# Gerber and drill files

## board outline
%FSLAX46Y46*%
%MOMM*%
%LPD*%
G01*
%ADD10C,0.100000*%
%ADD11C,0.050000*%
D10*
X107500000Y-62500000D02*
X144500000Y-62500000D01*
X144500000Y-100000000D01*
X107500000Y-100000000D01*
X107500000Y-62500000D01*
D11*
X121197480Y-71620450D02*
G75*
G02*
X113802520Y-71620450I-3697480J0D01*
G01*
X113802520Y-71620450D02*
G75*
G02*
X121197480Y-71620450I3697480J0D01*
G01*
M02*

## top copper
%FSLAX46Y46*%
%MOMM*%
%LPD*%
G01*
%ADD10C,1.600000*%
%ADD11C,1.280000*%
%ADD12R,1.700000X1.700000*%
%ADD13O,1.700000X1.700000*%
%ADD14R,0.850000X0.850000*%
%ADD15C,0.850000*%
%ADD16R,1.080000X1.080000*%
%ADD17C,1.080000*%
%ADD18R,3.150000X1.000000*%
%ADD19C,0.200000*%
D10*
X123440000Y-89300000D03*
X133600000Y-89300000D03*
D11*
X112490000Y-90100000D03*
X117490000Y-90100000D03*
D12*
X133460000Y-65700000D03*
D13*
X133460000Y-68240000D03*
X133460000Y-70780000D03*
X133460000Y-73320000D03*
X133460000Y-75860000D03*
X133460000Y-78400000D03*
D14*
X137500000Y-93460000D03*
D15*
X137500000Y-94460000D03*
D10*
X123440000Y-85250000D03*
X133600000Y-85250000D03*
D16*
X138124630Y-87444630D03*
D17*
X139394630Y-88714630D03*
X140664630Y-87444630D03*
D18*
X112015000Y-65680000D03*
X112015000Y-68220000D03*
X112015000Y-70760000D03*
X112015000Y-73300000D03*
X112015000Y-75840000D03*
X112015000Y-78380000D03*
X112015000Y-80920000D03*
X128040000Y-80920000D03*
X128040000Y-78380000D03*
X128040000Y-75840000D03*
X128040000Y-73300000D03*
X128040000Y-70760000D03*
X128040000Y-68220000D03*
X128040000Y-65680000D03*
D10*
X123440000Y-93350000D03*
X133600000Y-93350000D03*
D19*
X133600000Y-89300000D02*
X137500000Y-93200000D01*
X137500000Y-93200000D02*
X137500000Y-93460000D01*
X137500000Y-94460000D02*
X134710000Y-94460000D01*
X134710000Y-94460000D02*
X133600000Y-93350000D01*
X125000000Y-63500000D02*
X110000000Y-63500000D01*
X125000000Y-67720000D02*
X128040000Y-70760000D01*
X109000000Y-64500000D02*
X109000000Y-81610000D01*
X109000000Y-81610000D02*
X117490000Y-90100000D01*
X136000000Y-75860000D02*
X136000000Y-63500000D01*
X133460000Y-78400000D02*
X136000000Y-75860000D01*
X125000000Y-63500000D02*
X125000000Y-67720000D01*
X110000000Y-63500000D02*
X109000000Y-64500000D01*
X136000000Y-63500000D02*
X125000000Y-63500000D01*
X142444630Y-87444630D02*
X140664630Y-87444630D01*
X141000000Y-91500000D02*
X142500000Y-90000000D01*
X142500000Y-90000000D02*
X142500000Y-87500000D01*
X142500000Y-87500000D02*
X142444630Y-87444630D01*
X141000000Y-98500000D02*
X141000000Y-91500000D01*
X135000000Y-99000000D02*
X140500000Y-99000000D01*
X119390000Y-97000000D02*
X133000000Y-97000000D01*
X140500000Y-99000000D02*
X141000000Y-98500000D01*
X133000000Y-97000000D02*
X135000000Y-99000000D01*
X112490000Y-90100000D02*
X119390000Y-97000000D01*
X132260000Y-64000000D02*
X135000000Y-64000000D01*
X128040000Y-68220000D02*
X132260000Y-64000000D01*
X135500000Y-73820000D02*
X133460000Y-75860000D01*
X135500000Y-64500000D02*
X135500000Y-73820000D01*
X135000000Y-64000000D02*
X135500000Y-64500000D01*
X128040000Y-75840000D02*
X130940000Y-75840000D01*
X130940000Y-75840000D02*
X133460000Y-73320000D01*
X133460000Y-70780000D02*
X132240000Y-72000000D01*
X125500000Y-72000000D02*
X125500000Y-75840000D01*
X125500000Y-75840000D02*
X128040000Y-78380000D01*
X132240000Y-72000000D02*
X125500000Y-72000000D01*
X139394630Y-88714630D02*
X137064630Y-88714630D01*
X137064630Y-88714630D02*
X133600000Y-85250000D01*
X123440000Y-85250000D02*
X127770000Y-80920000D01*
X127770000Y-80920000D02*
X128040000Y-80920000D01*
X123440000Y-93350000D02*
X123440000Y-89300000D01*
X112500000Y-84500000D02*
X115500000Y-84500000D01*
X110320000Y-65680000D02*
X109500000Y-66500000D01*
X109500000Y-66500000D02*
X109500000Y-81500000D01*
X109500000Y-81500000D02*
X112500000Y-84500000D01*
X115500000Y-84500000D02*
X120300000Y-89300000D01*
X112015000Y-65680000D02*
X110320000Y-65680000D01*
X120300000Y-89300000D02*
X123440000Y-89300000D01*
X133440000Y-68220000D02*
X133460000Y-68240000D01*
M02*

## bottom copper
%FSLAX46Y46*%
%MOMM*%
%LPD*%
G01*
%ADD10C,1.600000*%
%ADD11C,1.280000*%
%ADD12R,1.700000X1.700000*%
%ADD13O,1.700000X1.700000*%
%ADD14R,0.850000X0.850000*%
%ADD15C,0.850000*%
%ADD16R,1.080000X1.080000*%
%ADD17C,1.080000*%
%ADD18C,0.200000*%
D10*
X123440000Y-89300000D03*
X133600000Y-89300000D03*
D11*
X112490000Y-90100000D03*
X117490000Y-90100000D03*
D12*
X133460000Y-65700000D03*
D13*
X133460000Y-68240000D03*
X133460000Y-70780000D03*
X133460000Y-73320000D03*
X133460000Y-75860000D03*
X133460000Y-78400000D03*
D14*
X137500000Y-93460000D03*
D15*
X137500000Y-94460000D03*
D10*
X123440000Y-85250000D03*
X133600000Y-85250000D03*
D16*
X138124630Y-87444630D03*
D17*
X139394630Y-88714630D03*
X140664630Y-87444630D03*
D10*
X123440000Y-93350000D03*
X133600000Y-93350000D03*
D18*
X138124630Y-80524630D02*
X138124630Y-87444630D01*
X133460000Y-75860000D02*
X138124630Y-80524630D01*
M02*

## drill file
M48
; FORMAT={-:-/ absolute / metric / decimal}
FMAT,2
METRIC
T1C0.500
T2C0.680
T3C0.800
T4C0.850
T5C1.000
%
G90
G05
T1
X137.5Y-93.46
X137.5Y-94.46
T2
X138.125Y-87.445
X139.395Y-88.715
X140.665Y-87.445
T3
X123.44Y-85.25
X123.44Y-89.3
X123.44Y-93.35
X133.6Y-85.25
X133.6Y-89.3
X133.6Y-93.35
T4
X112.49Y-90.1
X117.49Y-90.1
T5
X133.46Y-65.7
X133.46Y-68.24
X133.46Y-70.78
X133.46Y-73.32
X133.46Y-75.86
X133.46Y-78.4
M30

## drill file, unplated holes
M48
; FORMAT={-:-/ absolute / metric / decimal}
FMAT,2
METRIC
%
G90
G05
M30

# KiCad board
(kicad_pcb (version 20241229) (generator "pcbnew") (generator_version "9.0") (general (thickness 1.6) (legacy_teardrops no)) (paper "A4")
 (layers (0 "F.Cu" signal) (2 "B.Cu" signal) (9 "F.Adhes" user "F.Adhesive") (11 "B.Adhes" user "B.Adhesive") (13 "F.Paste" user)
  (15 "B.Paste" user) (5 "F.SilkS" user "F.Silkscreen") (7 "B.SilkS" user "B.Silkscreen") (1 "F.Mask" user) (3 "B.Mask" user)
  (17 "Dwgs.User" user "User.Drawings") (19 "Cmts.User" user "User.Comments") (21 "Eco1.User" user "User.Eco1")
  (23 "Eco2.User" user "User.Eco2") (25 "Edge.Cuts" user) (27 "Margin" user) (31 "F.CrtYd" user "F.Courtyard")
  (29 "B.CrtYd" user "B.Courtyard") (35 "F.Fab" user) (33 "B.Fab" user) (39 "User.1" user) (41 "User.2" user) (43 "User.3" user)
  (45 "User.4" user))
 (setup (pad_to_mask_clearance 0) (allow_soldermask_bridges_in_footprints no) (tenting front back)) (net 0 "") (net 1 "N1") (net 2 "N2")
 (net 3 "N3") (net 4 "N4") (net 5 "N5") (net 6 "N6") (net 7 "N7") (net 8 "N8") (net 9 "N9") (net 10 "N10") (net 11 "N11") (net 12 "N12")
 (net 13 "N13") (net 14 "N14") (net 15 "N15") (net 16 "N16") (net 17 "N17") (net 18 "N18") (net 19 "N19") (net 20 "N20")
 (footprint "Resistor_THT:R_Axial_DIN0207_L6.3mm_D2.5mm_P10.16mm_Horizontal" (layer "F.Cu") (at 123.44 89.3)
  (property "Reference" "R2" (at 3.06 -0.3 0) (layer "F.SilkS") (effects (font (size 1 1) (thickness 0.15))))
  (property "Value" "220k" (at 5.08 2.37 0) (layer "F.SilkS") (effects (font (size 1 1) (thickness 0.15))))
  (pad "1" thru_hole circle (at 0 0) (size 1.6 1.6) (drill 0.8) (layers "*.Cu" "*.Mask") (remove_unused_layers no) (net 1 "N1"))
  (pad "2" thru_hole circle (at 10.16 0) (size 1.6 1.6) (drill 0.8) (layers "*.Cu" "*.Mask") (remove_unused_layers no) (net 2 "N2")))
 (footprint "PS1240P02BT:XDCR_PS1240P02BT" (layer "F.Cu") (at 114.99 90.1)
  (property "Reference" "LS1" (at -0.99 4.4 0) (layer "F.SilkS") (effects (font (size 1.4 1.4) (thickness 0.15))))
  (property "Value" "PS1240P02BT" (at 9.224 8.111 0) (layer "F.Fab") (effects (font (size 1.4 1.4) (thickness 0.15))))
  (pad "1" thru_hole circle (at -2.5 0) (size 1.28 1.28) (drill 0.85) (layers "*.Cu" "*.Mask") (remove_unused_layers no) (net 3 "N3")
   (solder_mask_margin 0.102))
  (pad "2" thru_hole circle (at 2.5 0) (size 1.28 1.28) (drill 0.85) (layers "*.Cu" "*.Mask") (remove_unused_layers no) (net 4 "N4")
   (solder_mask_margin 0.102)))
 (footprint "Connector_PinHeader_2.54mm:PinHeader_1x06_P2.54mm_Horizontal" (layer "F.Cu") (at 133.46 65.7)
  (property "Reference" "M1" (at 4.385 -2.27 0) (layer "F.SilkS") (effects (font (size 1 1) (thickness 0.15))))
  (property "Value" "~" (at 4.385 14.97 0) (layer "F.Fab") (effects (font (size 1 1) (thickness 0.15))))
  (pad "1" thru_hole rect (at 0 0) (size 1.7 1.7) (drill 1) (layers "*.Cu" "*.Mask") (remove_unused_layers no) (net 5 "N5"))
  (pad "2" thru_hole oval (at 0 2.54) (size 1.7 1.7) (drill 1) (layers "*.Cu" "*.Mask") (remove_unused_layers no) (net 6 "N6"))
  (pad "3" thru_hole oval (at 0 5.08) (size 1.7 1.7) (drill 1) (layers "*.Cu" "*.Mask") (remove_unused_layers no) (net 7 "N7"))
  (pad "4" thru_hole oval (at 0 7.62) (size 1.7 1.7) (drill 1) (layers "*.Cu" "*.Mask") (remove_unused_layers no) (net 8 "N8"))
  (pad "5" thru_hole oval (at 0 10.16) (size 1.7 1.7) (drill 1) (layers "*.Cu" "*.Mask") (remove_unused_layers no) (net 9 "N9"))
  (pad "6" thru_hole oval (at 0 12.7) (size 1.7 1.7) (drill 1) (layers "*.Cu" "*.Mask") (remove_unused_layers no) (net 4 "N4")))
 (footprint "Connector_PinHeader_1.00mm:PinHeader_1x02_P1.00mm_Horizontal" (layer "F.Cu") (at 137.5 93.46)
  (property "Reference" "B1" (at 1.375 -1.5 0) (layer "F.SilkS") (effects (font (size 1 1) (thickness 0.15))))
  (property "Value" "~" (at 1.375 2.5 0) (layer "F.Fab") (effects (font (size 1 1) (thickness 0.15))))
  (pad "1" thru_hole rect (at 0 0) (size 0.85 0.85) (drill 0.5) (layers "*.Cu" "*.Mask") (remove_unused_layers no) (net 2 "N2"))
  (pad "2" thru_hole circle (at 0 1) (size 0.85 0.85) (drill 0.5) (layers "*.Cu" "*.Mask") (remove_unused_layers no) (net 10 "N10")))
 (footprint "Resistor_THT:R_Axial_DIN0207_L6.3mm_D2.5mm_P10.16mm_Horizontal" (layer "F.Cu") (at 123.44 85.25)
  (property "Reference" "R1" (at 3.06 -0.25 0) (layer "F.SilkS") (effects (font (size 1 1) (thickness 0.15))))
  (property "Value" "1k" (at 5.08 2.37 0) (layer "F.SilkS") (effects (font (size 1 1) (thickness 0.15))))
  (pad "1" thru_hole circle (at 0 0) (size 1.6 1.6) (drill 0.8) (layers "*.Cu" "*.Mask") (remove_unused_layers no) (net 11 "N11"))
  (pad "2" thru_hole circle (at 10.16 0) (size 1.6 1.6) (drill 0.8) (layers "*.Cu" "*.Mask") (remove_unused_layers no) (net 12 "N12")))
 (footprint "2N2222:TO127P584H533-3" (layer "F.Cu") (at 139.39463 87.44463)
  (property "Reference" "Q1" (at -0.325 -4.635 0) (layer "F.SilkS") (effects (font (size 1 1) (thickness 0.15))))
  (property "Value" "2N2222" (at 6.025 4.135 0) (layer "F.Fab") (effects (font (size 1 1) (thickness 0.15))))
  (pad "1" thru_hole rect (at -1.27 0) (size 1.08 1.08) (drill 0.68) (layers "*.Cu" "*.Mask") (remove_unused_layers no) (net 9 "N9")
   (solder_mask_margin 0.102))
  (pad "2" thru_hole circle (at 0 1.27) (size 1.08 1.08) (drill 0.68) (layers "*.Cu" "*.Mask") (remove_unused_layers no) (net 12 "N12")
   (solder_mask_margin 0.102))
  (pad "3" thru_hole circle (at 1.27 0 3) (size 1.08 1.08) (drill 0.68) (layers "*.Cu" "*.Mask") (remove_unused_layers no) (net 3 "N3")
   (solder_mask_margin 0.102)))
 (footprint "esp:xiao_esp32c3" (layer "F.Cu") (at 120.615 75.1)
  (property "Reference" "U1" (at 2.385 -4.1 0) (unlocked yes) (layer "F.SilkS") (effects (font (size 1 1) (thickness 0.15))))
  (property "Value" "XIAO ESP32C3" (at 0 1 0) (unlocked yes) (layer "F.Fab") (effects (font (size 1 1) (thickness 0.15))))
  (pad "1" smd rect (at -8.6 -9.42) (size 3.15 1) (layers "F.Cu" "F.Mask" "F.Paste") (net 1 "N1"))
  (pad "2" smd rect (at -8.6 -6.88) (size 3.15 1) (layers "F.Cu" "F.Mask" "F.Paste") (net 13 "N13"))
  (pad "3" smd rect (at -8.6 -4.34) (size 3.15 1) (layers "F.Cu" "F.Mask" "F.Paste") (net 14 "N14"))
  (pad "4" smd rect (at -8.6 -1.8) (size 3.15 1) (layers "F.Cu" "F.Mask" "F.Paste") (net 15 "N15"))
  (pad "5" smd rect (at -8.6 0.74) (size 3.15 1) (layers "F.Cu" "F.Mask" "F.Paste") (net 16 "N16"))
  (pad "6" smd rect (at -8.6 3.28) (size 3.15 1) (layers "F.Cu" "F.Mask" "F.Paste") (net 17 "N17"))
  (pad "7" smd rect (at -8.6 5.82) (size 3.15 1) (layers "F.Cu" "F.Mask" "F.Paste") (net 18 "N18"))
  (pad "8" smd rect (at 7.425 5.82) (size 3.15 1) (layers "F.Cu" "F.Mask" "F.Paste") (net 11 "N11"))
  (pad "9" smd rect (at 7.425 3.28) (size 3.15 1) (layers "F.Cu" "F.Mask" "F.Paste") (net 7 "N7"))
  (pad "10" smd rect (at 7.425 0.74) (size 3.15 1) (layers "F.Cu" "F.Mask" "F.Paste") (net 8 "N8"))
  (pad "11" smd rect (at 7.425 -1.8) (size 3.15 1) (layers "F.Cu" "F.Mask" "F.Paste") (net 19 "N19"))
  (pad "12" smd rect (at 7.425 -4.34) (size 3.15 1) (layers "F.Cu" "F.Mask" "F.Paste") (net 4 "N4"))
  (pad "13" smd rect (at 7.425 -6.88) (size 3.15 1) (layers "F.Cu" "F.Mask" "F.Paste") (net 9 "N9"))
  (pad "14" smd rect (at 7.425 -9.42) (size 3.15 1) (layers "F.Cu" "F.Mask" "F.Paste") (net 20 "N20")))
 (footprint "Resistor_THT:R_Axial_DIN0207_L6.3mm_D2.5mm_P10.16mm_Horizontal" (layer "F.Cu") (at 123.44 93.35)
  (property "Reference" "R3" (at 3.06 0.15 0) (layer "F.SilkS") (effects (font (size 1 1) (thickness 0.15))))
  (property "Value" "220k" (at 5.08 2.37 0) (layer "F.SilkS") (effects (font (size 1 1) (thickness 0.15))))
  (pad "1" thru_hole circle (at 0 0) (size 1.6 1.6) (drill 0.8) (layers "*.Cu" "*.Mask") (remove_unused_layers no) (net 1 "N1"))
  (pad "2" thru_hole circle (at 10.16 0) (size 1.6 1.6) (drill 0.8) (layers "*.Cu" "*.Mask") (remove_unused_layers no) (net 10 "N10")))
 (gr_rect (start 107.5 62.5) (end 144.5 100) (stroke (width 0.1) (type solid)) (fill no) (layer "Edge.Cuts"))
 (gr_circle (center 117.5 71.62045) (end 119 75) (stroke (width 0.05) (type default)) (fill no) (layer "Edge.Cuts"))
 (segment (start 133.6 89.3) (end 137.5 93.2) (width 0.2) (layer "F.Cu") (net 2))
 (segment (start 137.5 93.2) (end 137.5 93.46) (width 0.2) (layer "F.Cu") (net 2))
 (segment (start 137.5 94.46) (end 134.71 94.46) (width 0.2) (layer "F.Cu") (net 10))
 (segment (start 134.71 94.46) (end 133.6 93.35) (width 0.2) (layer "F.Cu") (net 10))
 (segment (start 125 63.5) (end 110 63.5) (width 0.2) (layer "F.Cu") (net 4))
 (segment (start 125 67.72) (end 128.04 70.76) (width 0.2) (layer "F.Cu") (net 4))
 (segment (start 109 64.5) (end 109 81.61) (width 0.2) (layer "F.Cu") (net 4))
 (segment (start 109 81.61) (end 117.49 90.1) (width 0.2) (layer "F.Cu") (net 4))
 (segment (start 136 75.86) (end 136 63.5) (width 0.2) (layer "F.Cu") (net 4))
 (segment (start 133.46 78.4) (end 136 75.86) (width 0.2) (layer "F.Cu") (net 4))
 (segment (start 125 63.5) (end 125 67.72) (width 0.2) (layer "F.Cu") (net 4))
 (segment (start 110 63.5) (end 109 64.5) (width 0.2) (layer "F.Cu") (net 4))
 (segment (start 136 63.5) (end 125 63.5) (width 0.2) (layer "F.Cu") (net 4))
 (segment (start 142.44463 87.44463) (end 140.66463 87.44463) (width 0.2) (layer "F.Cu") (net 3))
 (segment (start 141 91.5) (end 142.5 90) (width 0.2) (layer "F.Cu") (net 3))
 (segment (start 142.5 90) (end 142.5 87.5) (width 0.2) (layer "F.Cu") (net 3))
 (segment (start 142.5 87.5) (end 142.44463 87.44463) (width 0.2) (layer "F.Cu") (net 3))
 (segment (start 141 98.5) (end 141 91.5) (width 0.2) (layer "F.Cu") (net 3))
 (segment (start 135 99) (end 140.5 99) (width 0.2) (layer "F.Cu") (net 3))
 (segment (start 119.39 97) (end 133 97) (width 0.2) (layer "F.Cu") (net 3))
 (segment (start 140.5 99) (end 141 98.5) (width 0.2) (layer "F.Cu") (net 3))
 (segment (start 133 97) (end 135 99) (width 0.2) (layer "F.Cu") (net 3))
 (segment (start 112.49 90.1) (end 119.39 97) (width 0.2) (layer "F.Cu") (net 3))
 (segment (start 132.26 64) (end 135 64) (width 0.2) (layer "F.Cu") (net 9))
 (segment (start 128.04 68.22) (end 132.26 64) (width 0.2) (layer "F.Cu") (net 9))
 (segment (start 135.5 73.82) (end 133.46 75.86) (width 0.2) (layer "F.Cu") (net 9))
 (segment (start 135.5 64.5) (end 135.5 73.82) (width 0.2) (layer "F.Cu") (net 9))
 (segment (start 135 64) (end 135.5 64.5) (width 0.2) (layer "F.Cu") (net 9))
 (segment (start 138.12463 80.52463) (end 138.12463 87.44463) (width 0.2) (layer "B.Cu") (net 9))
 (segment (start 133.46 75.86) (end 138.12463 80.52463) (width 0.2) (layer "B.Cu") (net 9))
 (segment (start 128.04 75.84) (end 130.94 75.84) (width 0.2) (layer "F.Cu") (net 8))
 (segment (start 130.94 75.84) (end 133.46 73.32) (width 0.2) (layer "F.Cu") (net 8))
 (segment (start 133.46 70.78) (end 132.24 72) (width 0.2) (layer "F.Cu") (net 7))
 (segment (start 125.5 72) (end 125.5 75.84) (width 0.2) (layer "F.Cu") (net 7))
 (segment (start 125.5 75.84) (end 128.04 78.38) (width 0.2) (layer "F.Cu") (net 7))
 (segment (start 132.24 72) (end 125.5 72) (width 0.2) (layer "F.Cu") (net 7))
 (segment (start 139.39463 88.71463) (end 137.06463 88.71463) (width 0.2) (layer "F.Cu") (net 12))
 (segment (start 137.06463 88.71463) (end 133.6 85.25) (width 0.2) (layer "F.Cu") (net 12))
 (segment (start 123.44 85.25) (end 127.77 80.92) (width 0.2) (layer "F.Cu") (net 11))
 (segment (start 127.77 80.92) (end 128.04 80.92) (width 0.2) (layer "F.Cu") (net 11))
 (segment (start 123.44 93.35) (end 123.44 89.3) (width 0.2) (layer "F.Cu") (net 1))
 (segment (start 112.5 84.5) (end 115.5 84.5) (width 0.2) (layer "F.Cu") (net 1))
 (segment (start 110.32 65.68) (end 109.5 66.5) (width 0.2) (layer "F.Cu") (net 1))
 (segment (start 109.5 66.5) (end 109.5 81.5) (width 0.2) (layer "F.Cu") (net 1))
 (segment (start 109.5 81.5) (end 112.5 84.5) (width 0.2) (layer "F.Cu") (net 1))
 (segment (start 115.5 84.5) (end 120.3 89.3) (width 0.2) (layer "F.Cu") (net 1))
 (segment (start 112.015 65.68) (end 110.32 65.68) (width 0.2) (layer "F.Cu") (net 1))
 (segment (start 120.3 89.3) (end 123.44 89.3) (width 0.2) (layer "F.Cu") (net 1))
 (segment (start 133.44 68.22) (end 133.46 68.24) (width 0.2) (layer "F.Cu") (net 6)))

